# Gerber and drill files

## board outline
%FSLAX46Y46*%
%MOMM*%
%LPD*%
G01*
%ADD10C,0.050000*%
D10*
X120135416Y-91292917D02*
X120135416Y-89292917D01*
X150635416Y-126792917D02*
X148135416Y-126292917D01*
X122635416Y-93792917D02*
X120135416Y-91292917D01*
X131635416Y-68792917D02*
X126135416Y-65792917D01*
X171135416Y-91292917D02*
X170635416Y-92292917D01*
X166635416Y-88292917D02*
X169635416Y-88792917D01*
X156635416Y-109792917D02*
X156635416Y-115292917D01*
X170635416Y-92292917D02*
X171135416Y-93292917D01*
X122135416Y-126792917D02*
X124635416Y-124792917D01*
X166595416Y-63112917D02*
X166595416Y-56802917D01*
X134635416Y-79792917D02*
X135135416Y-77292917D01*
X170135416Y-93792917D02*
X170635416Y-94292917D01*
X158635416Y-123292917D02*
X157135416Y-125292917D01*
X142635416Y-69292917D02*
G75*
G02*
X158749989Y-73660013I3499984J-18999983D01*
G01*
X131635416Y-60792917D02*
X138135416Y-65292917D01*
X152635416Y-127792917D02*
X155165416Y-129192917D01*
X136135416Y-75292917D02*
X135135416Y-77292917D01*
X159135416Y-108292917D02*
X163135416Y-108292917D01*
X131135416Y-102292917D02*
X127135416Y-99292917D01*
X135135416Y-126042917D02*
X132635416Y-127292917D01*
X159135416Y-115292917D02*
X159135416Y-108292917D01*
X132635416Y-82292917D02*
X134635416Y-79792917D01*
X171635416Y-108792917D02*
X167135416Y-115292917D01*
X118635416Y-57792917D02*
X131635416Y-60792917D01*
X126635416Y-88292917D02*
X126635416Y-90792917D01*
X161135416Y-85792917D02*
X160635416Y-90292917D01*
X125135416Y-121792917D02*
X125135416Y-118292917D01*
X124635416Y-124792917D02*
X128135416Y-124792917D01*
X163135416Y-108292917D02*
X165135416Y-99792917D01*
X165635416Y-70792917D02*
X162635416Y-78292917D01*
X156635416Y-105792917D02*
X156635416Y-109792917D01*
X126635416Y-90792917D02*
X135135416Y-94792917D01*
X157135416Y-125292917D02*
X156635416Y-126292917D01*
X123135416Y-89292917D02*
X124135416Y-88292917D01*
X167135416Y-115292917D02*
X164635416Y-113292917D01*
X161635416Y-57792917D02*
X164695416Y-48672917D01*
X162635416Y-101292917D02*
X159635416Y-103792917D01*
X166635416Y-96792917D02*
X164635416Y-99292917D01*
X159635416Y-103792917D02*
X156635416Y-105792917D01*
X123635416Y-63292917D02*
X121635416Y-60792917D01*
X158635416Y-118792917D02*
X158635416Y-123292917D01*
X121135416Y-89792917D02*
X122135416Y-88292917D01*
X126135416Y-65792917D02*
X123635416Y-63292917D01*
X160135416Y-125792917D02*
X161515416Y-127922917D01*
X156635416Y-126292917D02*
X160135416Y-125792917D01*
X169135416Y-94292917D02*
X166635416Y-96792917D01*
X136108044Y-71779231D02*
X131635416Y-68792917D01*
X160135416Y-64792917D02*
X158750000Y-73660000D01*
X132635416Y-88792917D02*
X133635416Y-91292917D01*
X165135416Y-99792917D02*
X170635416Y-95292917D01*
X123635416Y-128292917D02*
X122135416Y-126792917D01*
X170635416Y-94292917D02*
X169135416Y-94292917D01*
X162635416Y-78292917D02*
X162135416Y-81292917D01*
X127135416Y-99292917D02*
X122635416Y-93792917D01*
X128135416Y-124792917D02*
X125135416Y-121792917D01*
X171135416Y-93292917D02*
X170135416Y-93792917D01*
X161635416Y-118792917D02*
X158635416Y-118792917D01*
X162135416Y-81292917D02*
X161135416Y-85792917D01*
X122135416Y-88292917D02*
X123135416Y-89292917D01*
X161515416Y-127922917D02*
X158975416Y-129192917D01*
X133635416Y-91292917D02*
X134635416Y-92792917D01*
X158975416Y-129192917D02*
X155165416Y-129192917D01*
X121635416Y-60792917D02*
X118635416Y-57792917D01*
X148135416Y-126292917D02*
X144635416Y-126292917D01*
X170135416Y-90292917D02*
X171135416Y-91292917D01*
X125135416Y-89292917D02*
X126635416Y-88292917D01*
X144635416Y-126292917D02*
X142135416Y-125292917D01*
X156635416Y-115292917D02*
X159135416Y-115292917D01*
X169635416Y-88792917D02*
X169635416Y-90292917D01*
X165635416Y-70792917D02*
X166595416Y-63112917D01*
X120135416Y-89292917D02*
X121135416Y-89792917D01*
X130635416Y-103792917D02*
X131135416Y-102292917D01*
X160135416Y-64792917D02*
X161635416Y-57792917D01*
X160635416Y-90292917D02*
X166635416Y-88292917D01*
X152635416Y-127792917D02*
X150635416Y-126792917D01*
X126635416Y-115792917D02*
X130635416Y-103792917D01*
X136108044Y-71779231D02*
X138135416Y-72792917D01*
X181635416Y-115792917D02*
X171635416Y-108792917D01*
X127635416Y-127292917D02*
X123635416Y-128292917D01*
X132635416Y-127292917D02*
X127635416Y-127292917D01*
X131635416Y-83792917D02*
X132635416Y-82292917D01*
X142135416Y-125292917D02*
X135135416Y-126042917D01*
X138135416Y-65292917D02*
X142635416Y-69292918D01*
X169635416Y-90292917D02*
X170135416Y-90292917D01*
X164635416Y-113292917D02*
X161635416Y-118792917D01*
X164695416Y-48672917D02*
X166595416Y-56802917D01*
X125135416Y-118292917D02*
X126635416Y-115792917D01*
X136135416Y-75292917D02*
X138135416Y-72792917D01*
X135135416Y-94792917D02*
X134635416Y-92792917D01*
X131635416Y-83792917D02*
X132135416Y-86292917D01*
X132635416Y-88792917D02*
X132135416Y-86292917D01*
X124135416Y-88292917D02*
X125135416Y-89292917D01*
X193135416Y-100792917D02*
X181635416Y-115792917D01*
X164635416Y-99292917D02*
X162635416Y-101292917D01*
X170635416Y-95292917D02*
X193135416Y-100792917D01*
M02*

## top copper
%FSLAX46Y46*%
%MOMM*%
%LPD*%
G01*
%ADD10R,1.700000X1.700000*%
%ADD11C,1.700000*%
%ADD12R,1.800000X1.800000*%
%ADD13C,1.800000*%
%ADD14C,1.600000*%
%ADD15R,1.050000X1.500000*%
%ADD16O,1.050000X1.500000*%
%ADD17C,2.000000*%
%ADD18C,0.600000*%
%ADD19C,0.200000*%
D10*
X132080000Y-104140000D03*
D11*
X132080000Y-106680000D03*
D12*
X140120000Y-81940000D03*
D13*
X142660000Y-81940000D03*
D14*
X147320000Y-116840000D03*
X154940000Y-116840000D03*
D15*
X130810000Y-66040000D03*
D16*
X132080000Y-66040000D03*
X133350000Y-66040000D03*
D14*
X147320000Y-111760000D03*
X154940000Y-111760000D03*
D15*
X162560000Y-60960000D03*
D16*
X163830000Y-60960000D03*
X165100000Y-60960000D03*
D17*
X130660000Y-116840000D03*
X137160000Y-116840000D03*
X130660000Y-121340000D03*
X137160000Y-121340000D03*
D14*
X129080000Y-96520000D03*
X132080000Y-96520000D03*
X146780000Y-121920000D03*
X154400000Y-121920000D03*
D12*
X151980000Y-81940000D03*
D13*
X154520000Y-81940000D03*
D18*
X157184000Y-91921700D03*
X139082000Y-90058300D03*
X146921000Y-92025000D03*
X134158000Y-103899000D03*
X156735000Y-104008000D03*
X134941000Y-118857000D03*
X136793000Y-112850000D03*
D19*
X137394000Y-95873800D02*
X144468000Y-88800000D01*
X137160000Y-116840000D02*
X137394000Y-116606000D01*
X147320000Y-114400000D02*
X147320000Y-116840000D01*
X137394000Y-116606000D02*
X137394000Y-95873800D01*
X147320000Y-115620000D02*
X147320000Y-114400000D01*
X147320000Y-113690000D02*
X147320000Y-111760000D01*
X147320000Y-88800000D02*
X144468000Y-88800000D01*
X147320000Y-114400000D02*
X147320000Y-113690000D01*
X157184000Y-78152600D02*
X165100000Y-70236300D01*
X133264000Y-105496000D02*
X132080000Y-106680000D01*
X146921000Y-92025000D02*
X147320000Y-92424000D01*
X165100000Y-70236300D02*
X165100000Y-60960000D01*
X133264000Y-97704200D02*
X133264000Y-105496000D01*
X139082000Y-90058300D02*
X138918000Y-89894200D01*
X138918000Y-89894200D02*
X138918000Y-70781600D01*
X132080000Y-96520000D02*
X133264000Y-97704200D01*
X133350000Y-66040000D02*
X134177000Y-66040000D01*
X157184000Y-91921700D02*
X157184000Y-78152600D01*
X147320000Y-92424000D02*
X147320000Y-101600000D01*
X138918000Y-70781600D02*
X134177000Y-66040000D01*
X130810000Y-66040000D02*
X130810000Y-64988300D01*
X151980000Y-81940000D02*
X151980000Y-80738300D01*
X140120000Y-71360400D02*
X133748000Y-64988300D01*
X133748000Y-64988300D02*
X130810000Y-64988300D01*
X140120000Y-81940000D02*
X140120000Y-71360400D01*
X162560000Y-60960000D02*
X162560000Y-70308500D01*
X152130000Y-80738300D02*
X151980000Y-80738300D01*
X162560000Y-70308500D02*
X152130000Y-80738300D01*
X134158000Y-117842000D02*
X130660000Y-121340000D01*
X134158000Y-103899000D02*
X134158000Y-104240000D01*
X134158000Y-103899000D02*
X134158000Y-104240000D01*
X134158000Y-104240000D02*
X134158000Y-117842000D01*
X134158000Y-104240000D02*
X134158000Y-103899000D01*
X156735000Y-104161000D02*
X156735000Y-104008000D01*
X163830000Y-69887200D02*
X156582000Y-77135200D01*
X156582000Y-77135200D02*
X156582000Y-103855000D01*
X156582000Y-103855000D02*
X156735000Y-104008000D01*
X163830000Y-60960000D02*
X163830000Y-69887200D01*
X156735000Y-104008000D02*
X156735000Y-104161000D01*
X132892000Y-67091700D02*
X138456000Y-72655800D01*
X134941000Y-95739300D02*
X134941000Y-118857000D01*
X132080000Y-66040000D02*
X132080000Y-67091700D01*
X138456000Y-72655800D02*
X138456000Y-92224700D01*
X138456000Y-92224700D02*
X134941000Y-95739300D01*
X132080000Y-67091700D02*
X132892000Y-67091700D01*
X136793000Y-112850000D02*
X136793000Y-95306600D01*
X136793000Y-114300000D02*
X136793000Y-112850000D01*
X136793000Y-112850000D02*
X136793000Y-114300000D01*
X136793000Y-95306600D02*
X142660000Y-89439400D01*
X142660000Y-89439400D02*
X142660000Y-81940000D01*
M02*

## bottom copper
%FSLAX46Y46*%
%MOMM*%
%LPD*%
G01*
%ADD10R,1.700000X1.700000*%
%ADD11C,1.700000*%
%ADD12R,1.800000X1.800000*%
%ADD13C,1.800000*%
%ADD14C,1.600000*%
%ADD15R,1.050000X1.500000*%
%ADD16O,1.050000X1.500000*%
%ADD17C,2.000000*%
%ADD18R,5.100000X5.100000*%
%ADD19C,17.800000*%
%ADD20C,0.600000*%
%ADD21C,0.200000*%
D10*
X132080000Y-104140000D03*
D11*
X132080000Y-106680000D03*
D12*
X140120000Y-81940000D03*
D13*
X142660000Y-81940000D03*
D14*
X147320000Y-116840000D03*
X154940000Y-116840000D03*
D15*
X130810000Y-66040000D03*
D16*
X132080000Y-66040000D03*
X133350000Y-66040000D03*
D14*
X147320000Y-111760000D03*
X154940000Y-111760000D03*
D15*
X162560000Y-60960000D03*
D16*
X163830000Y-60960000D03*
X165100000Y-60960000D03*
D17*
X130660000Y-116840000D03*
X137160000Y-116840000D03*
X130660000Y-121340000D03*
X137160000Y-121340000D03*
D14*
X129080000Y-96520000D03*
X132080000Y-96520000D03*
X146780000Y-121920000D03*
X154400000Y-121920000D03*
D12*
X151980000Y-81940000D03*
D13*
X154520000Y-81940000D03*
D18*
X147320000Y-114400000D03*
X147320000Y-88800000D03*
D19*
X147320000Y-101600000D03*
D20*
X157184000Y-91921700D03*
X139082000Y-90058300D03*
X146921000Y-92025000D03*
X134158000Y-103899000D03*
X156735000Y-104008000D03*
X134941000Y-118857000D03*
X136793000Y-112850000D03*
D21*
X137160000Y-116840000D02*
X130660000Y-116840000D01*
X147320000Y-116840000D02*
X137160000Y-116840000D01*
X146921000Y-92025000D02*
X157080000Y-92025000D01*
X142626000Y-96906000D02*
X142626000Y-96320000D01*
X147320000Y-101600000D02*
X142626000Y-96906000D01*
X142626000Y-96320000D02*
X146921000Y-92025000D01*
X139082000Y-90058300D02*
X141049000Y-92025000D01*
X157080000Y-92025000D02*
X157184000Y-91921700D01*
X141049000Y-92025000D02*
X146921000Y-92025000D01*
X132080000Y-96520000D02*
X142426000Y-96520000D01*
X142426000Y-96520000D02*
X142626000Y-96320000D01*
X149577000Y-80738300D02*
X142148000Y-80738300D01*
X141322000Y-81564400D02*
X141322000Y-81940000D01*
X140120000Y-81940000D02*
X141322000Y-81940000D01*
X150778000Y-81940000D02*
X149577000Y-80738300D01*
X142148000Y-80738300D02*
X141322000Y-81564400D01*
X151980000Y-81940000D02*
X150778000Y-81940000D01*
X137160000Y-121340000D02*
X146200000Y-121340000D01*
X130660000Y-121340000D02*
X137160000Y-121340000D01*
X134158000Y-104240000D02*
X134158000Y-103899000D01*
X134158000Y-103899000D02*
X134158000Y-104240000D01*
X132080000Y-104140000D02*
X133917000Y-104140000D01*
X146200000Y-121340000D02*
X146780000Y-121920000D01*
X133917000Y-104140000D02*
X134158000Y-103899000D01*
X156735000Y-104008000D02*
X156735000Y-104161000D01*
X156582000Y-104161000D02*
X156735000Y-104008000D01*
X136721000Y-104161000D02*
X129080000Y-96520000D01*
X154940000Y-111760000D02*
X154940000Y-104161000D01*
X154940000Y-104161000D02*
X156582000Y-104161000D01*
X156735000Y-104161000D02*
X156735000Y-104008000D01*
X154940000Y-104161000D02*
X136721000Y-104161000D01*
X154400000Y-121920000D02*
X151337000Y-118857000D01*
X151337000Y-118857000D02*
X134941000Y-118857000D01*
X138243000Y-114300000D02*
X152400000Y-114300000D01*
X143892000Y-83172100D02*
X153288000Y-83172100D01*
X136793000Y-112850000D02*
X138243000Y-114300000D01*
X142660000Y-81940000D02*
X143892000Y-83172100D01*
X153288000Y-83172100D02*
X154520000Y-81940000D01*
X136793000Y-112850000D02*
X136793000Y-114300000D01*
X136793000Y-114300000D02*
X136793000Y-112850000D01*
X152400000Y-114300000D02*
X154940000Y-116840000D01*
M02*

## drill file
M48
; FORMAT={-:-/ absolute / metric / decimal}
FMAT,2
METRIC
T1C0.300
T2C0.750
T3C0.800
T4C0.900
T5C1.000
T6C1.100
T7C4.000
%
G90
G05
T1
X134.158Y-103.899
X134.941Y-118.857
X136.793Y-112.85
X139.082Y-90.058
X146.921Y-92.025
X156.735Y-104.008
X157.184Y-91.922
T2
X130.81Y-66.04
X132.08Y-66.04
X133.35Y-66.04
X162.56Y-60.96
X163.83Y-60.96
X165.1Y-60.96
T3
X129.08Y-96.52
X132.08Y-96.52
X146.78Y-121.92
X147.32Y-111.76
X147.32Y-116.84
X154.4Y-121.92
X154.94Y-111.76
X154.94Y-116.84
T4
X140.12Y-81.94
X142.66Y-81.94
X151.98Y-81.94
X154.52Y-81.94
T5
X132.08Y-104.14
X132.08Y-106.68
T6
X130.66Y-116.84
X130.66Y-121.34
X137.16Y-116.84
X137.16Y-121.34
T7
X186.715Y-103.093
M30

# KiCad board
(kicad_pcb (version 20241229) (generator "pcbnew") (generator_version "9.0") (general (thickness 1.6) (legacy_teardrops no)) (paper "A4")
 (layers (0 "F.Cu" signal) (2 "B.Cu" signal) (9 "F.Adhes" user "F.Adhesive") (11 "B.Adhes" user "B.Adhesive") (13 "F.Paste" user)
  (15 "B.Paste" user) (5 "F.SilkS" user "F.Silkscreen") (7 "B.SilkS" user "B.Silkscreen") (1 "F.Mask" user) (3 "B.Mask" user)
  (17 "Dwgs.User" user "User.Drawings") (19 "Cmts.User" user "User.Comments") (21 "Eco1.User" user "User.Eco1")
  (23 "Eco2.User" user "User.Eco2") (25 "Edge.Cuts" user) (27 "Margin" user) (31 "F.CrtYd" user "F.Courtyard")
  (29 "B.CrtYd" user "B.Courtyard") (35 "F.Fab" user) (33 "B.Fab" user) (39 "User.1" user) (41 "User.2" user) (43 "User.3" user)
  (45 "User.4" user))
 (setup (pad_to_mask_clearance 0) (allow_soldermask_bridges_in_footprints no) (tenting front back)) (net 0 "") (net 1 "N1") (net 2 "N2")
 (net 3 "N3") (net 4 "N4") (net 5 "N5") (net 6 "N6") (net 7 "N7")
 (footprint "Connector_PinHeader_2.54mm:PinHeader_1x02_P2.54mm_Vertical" (layer "F.Cu") (at 132.08 104.14)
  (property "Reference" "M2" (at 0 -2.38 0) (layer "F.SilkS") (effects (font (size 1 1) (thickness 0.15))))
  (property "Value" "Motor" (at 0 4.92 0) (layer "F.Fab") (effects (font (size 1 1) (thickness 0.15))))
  (pad "1" thru_hole rect (at 0 0) (size 1.7 1.7) (drill 1) (layers "*.Cu" "*.Mask") (remove_unused_layers no) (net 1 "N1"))
  (pad "2" thru_hole circle (at 0 2.54) (size 1.7 1.7) (drill 1) (layers "*.Cu" "*.Mask") (remove_unused_layers no) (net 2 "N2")))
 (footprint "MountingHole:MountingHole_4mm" (layer "F.Cu") (at 186.7154 103.0929)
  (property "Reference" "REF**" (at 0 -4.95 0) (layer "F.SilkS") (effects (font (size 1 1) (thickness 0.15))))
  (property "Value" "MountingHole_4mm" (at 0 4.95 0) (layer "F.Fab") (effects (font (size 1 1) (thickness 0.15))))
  (pad "" np_thru_hole circle (at 0 0) (size 4 4) (drill 4) (layers "*.Cu" "*.Mask")))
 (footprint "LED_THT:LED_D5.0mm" (layer "F.Cu") (at 140.12 81.94)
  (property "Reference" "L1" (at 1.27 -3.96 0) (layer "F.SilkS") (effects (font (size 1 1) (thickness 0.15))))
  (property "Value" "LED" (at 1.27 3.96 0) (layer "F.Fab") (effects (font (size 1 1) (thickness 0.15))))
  (pad "1" thru_hole rect (at 0 0) (size 1.8 1.8) (drill 0.9) (layers "*.Cu" "*.Mask") (remove_unused_layers no) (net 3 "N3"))
  (pad "2" thru_hole circle (at 2.54 0) (size 1.8 1.8) (drill 0.9) (layers "*.Cu" "*.Mask") (remove_unused_layers no) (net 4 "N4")))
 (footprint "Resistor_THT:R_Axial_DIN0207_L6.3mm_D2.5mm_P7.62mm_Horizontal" (layer "F.Cu") (at 147.32 116.84)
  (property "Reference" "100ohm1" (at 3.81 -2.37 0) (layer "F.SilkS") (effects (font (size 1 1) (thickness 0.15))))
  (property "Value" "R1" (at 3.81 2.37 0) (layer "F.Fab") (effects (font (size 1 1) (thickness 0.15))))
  (pad "1" thru_hole circle (at 0 0) (size 1.6 1.6) (drill 0.8) (layers "*.Cu" "*.Mask") (remove_unused_layers no) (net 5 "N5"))
  (pad "2" thru_hole circle (at 7.62 0) (size 1.6 1.6) (drill 0.8) (layers "*.Cu" "*.Mask") (remove_unused_layers no) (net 4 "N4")))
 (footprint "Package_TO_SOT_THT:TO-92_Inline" (layer "F.Cu") (at 130.81 66.04)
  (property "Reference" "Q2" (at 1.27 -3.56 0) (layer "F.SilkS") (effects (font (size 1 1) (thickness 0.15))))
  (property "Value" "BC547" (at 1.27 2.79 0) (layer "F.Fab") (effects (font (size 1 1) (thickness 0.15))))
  (pad "1" thru_hole rect (at 0 0) (size 1.05 1.5) (drill 0.75) (layers "*.Cu" "*.Mask") (remove_unused_layers no) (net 3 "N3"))
  (pad "2" thru_hole oval (at 1.27 0) (size 1.05 1.5) (drill 0.75) (layers "*.Cu" "*.Mask") (remove_unused_layers no) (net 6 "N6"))
  (pad "3" thru_hole oval (at 2.54 0) (size 1.05 1.5) (drill 0.75) (layers "*.Cu" "*.Mask") (remove_unused_layers no) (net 2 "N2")))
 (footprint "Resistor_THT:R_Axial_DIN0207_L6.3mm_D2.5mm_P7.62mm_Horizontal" (layer "F.Cu") (at 147.32 111.76)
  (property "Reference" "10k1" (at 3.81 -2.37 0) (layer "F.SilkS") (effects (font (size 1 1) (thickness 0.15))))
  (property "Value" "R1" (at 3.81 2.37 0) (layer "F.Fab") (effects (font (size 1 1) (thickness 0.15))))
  (pad "1" thru_hole circle (at 0 0) (size 1.6 1.6) (drill 0.8) (layers "*.Cu" "*.Mask") (remove_unused_layers no) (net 5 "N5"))
  (pad "2" thru_hole circle (at 7.62 0) (size 1.6 1.6) (drill 0.8) (layers "*.Cu" "*.Mask") (remove_unused_layers no) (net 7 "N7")))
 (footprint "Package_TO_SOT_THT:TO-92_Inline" (layer "F.Cu") (at 162.56 60.96)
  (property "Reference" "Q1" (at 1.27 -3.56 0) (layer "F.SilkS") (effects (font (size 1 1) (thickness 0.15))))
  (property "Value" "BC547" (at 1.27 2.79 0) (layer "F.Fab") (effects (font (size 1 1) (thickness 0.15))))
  (pad "1" thru_hole rect (at 0 0) (size 1.05 1.5) (drill 0.75) (layers "*.Cu" "*.Mask") (remove_unused_layers no) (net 3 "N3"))
  (pad "2" thru_hole oval (at 1.27 0) (size 1.05 1.5) (drill 0.75) (layers "*.Cu" "*.Mask") (remove_unused_layers no) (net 7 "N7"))
  (pad "3" thru_hole oval (at 2.54 0) (size 1.05 1.5) (drill 0.75) (layers "*.Cu" "*.Mask") (remove_unused_layers no) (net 2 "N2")))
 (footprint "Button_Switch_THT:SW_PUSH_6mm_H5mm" (layer "F.Cu") (at 130.66 116.84)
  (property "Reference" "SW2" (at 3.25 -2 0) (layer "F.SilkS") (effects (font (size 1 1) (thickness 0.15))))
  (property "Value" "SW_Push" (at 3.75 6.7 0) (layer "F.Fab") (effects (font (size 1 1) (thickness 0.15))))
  (pad "1" thru_hole circle (at 0 0 90) (size 2 2) (drill 1.1) (layers "*.Cu" "*.Mask") (remove_unused_layers no) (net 5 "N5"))
  (pad "1" thru_hole circle (at 6.5 0 90) (size 2 2) (drill 1.1) (layers "*.Cu" "*.Mask") (remove_unused_layers no) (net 5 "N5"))
  (pad "2" thru_hole circle (at 0 4.5 90) (size 2 2) (drill 1.1) (layers "*.Cu" "*.Mask") (remove_unused_layers no) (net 1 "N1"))
  (pad "2" thru_hole circle (at 6.5 4.5 90) (size 2 2) (drill 1.1) (layers "*.Cu" "*.Mask") (remove_unused_layers no) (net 1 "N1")))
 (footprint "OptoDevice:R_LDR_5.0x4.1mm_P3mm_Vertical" (layer "F.Cu") (at 129.08 96.52)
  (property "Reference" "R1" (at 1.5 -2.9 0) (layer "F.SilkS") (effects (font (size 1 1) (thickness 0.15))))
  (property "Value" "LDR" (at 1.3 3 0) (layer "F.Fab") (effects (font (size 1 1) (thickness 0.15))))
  (pad "1" thru_hole circle (at 0 0) (size 1.6 1.6) (drill 0.8) (layers "*.Cu" "*.Mask") (remove_unused_layers no) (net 7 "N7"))
  (pad "2" thru_hole circle (at 3 0) (size 1.6 1.6) (drill 0.8) (layers "*.Cu" "*.Mask") (remove_unused_layers no) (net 2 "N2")))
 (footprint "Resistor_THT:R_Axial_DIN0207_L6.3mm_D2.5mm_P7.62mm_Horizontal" (layer "F.Cu") (at 146.78 121.92)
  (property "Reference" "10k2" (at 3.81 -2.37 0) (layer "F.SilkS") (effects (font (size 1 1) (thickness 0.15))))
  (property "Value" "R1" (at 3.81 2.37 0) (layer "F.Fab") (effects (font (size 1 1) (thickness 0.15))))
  (pad "1" thru_hole circle (at 0 0) (size 1.6 1.6) (drill 0.8) (layers "*.Cu" "*.Mask") (remove_unused_layers no) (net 1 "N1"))
  (pad "2" thru_hole circle (at 7.62 0) (size 1.6 1.6) (drill 0.8) (layers "*.Cu" "*.Mask") (remove_unused_layers no) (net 6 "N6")))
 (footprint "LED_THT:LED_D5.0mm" (layer "F.Cu") (at 151.98 81.94)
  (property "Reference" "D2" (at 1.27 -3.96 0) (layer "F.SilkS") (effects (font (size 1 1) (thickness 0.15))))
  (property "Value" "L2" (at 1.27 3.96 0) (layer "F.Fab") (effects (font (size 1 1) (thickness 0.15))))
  (pad "1" thru_hole rect (at 0 0) (size 1.8 1.8) (drill 0.9) (layers "*.Cu" "*.Mask") (remove_unused_layers no) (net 3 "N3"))
  (pad "2" thru_hole circle (at 2.54 0) (size 1.8 1.8) (drill 0.9) (layers "*.Cu" "*.Mask") (remove_unused_layers no) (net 4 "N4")))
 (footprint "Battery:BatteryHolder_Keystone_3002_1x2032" (layer "B.Cu") (at 147.32 101.6 90)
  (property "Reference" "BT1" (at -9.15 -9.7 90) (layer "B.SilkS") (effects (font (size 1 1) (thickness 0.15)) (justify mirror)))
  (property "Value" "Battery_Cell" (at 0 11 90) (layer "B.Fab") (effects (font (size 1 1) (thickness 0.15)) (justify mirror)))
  (pad "1" smd rect (at -12.8 0 90) (size 5.1 5.1) (layers "B.Cu" "B.Mask" "B.Paste") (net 5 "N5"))
  (pad "1" smd rect (at 12.8 0 90) (size 5.1 5.1) (layers "B.Cu" "B.Mask" "B.Paste") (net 5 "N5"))
  (pad "2" smd circle (at 0 0 90) (size 17.8 17.8) (layers "B.Cu" "B.Mask") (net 2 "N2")))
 (gr_line (start 120.135416 91.292917) (end 120.135416 89.292917) (stroke (width 0.05) (type default)) (layer "Edge.Cuts"))
 (gr_line (start 150.635416 126.792917) (end 148.135416 126.292917) (stroke (width 0.05) (type default)) (layer "Edge.Cuts"))
 (gr_line (start 122.635416 93.792917) (end 120.135416 91.292917) (stroke (width 0.05) (type default)) (layer "Edge.Cuts"))
 (gr_line (start 131.635416 68.792917) (end 126.135416 65.792917) (stroke (width 0.05) (type default)) (layer "Edge.Cuts"))
 (gr_line (start 171.135416 91.292917) (end 170.635416 92.292917) (stroke (width 0.05) (type default)) (layer "Edge.Cuts"))
 (gr_line (start 166.635416 88.292917) (end 169.635416 88.792917) (stroke (width 0.05) (type default)) (layer "Edge.Cuts"))
 (gr_line (start 156.635416 109.792917) (end 156.635416 115.292917) (stroke (width 0.05) (type default)) (layer "Edge.Cuts"))
 (gr_line (start 170.635416 92.292917) (end 171.135416 93.292917) (stroke (width 0.05) (type default)) (layer "Edge.Cuts"))
 (gr_line (start 122.135416 126.792917) (end 124.635416 124.792917) (stroke (width 0.05) (type default)) (layer "Edge.Cuts"))
 (gr_line (start 166.595416 63.112917) (end 166.595416 56.802917) (stroke (width 0.05) (type default)) (layer "Edge.Cuts"))
 (gr_line (start 134.635416 79.792917) (end 135.135416 77.292917) (stroke (width 0.05) (type default)) (layer "Edge.Cuts"))
 (gr_line (start 170.135416 93.792917) (end 170.635416 94.292917) (stroke (width 0.05) (type default)) (layer "Edge.Cuts"))
 (gr_line (start 158.635416 123.292917) (end 157.135416 125.292917) (stroke (width 0.05) (type default)) (layer "Edge.Cuts"))
 (gr_arc (start 142.635416 69.292917) (mid 151.188807 69.645847) (end 158.75 73.66) (stroke (width 0.05) (type default)) (layer "Edge.Cuts"))
 (gr_line (start 131.635416 60.792917) (end 138.135416 65.292917) (stroke (width 0.05) (type default)) (layer "Edge.Cuts"))
 (gr_line (start 152.635416 127.792917) (end 155.165416 129.192917) (stroke (width 0.05) (type default)) (layer "Edge.Cuts"))
 (gr_line (start 136.135416 75.292917) (end 135.135416 77.292917) (stroke (width 0.05) (type default)) (layer "Edge.Cuts"))
 (gr_line (start 159.135416 108.292917) (end 163.135416 108.292917) (stroke (width 0.05) (type default)) (layer "Edge.Cuts"))
 (gr_line (start 131.135416 102.292917) (end 127.135416 99.292917) (stroke (width 0.05) (type default)) (layer "Edge.Cuts"))
 (gr_line (start 135.135416 126.042917) (end 132.635416 127.292917) (stroke (width 0.05) (type default)) (layer "Edge.Cuts"))
 (gr_line (start 159.135416 115.292917) (end 159.135416 108.292917) (stroke (width 0.05) (type default)) (layer "Edge.Cuts"))
 (gr_line (start 132.635416 82.292917) (end 134.635416 79.792917) (stroke (width 0.05) (type default)) (layer "Edge.Cuts"))
 (gr_line (start 171.635416 108.792917) (end 167.135416 115.292917) (stroke (width 0.05) (type default)) (layer "Edge.Cuts"))
 (gr_line (start 118.635416 57.792917) (end 131.635416 60.792917) (stroke (width 0.05) (type default)) (layer "Edge.Cuts"))
 (gr_line (start 126.635416 88.292917) (end 126.635416 90.792917) (stroke (width 0.05) (type default)) (layer "Edge.Cuts"))
 (gr_line (start 161.135416 85.792917) (end 160.635416 90.292917) (stroke (width 0.05) (type default)) (layer "Edge.Cuts"))
 (gr_line (start 125.135416 121.792917) (end 125.135416 118.292917) (stroke (width 0.05) (type default)) (layer "Edge.Cuts"))
 (gr_line (start 124.635416 124.792917) (end 128.135416 124.792917) (stroke (width 0.05) (type default)) (layer "Edge.Cuts"))
 (gr_line (start 163.135416 108.292917) (end 165.135416 99.792917) (stroke (width 0.05) (type default)) (layer "Edge.Cuts"))
 (gr_line (start 165.635416 70.792917) (end 162.635416 78.292917) (stroke (width 0.05) (type default)) (layer "Edge.Cuts"))
 (gr_line (start 156.635416 105.792917) (end 156.635416 109.792917) (stroke (width 0.05) (type default)) (layer "Edge.Cuts"))
 (gr_line (start 126.635416 90.792917) (end 135.135416 94.792917) (stroke (width 0.05) (type default)) (layer "Edge.Cuts"))
 (gr_line (start 157.135416 125.292917) (end 156.635416 126.292917) (stroke (width 0.05) (type default)) (layer "Edge.Cuts"))
 (gr_line (start 123.135416 89.292917) (end 124.135416 88.292917) (stroke (width 0.05) (type default)) (layer "Edge.Cuts"))
 (gr_line (start 167.135416 115.292917) (end 164.635416 113.292917) (stroke (width 0.05) (type default)) (layer "Edge.Cuts"))
 (gr_line (start 161.635416 57.792917) (end 164.695416 48.672917) (stroke (width 0.05) (type default)) (layer "Edge.Cuts"))
 (gr_line (start 162.635416 101.292917) (end 159.635416 103.792917) (stroke (width 0.05) (type default)) (layer "Edge.Cuts"))
 (gr_line (start 166.635416 96.792917) (end 164.635416 99.292917) (stroke (width 0.05) (type default)) (layer "Edge.Cuts"))
 (gr_line (start 159.635416 103.792917) (end 156.635416 105.792917) (stroke (width 0.05) (type default)) (layer "Edge.Cuts"))
 (gr_line (start 123.635416 63.292917) (end 121.635416 60.792917) (stroke (width 0.05) (type default)) (layer "Edge.Cuts"))
 (gr_line (start 158.635416 118.792917) (end 158.635416 123.292917) (stroke (width 0.05) (type default)) (layer "Edge.Cuts"))
 (gr_line (start 121.135416 89.792917) (end 122.135416 88.292917) (stroke (width 0.05) (type default)) (layer "Edge.Cuts"))
 (gr_line (start 126.135416 65.792917) (end 123.635416 63.292917) (stroke (width 0.05) (type default)) (layer "Edge.Cuts"))
 (gr_line (start 160.135416 125.792917) (end 161.515416 127.922917) (stroke (width 0.05) (type default)) (layer "Edge.Cuts"))
 (gr_line (start 156.635416 126.292917) (end 160.135416 125.792917) (stroke (width 0.05) (type default)) (layer "Edge.Cuts"))
 (gr_line (start 169.135416 94.292917) (end 166.635416 96.792917) (stroke (width 0.05) (type default)) (layer "Edge.Cuts"))
 (gr_line (start 136.108044 71.779231) (end 131.635416 68.792917) (stroke (width 0.05) (type default)) (layer "Edge.Cuts"))
 (gr_line (start 160.135416 64.792917) (end 158.75 73.66) (stroke (width 0.05) (type default)) (layer "Edge.Cuts"))
 (gr_line (start 132.635416 88.792917) (end 133.635416 91.292917) (stroke (width 0.05) (type default)) (layer "Edge.Cuts"))
 (gr_line (start 165.135416 99.792917) (end 170.635416 95.292917) (stroke (width 0.05) (type default)) (layer "Edge.Cuts"))
 (gr_line (start 123.635416 128.292917) (end 122.135416 126.792917) (stroke (width 0.05) (type default)) (layer "Edge.Cuts"))
 (gr_line (start 170.635416 94.292917) (end 169.135416 94.292917) (stroke (width 0.05) (type default)) (layer "Edge.Cuts"))
 (gr_line (start 162.635416 78.292917) (end 162.135416 81.292917) (stroke (width 0.05) (type default)) (layer "Edge.Cuts"))
 (gr_line (start 127.135416 99.292917) (end 122.635416 93.792917) (stroke (width 0.05) (type default)) (layer "Edge.Cuts"))
 (gr_line (start 128.135416 124.792917) (end 125.135416 121.792917) (stroke (width 0.05) (type default)) (layer "Edge.Cuts"))
 (gr_line (start 171.135416 93.292917) (end 170.135416 93.792917) (stroke (width 0.05) (type default)) (layer "Edge.Cuts"))
 (gr_line (start 161.635416 118.792917) (end 158.635416 118.792917) (stroke (width 0.05) (type default)) (layer "Edge.Cuts"))
 (gr_line (start 162.135416 81.292917) (end 161.135416 85.792917) (stroke (width 0.05) (type default)) (layer "Edge.Cuts"))
 (gr_line (start 122.135416 88.292917) (end 123.135416 89.292917) (stroke (width 0.05) (type default)) (layer "Edge.Cuts"))
 (gr_line (start 161.515416 127.922917) (end 158.975416 129.192917) (stroke (width 0.05) (type default)) (layer "Edge.Cuts"))
 (gr_line (start 133.635416 91.292917) (end 134.635416 92.792917) (stroke (width 0.05) (type default)) (layer "Edge.Cuts"))
 (gr_line (start 158.975416 129.192917) (end 155.165416 129.192917) (stroke (width 0.05) (type default)) (layer "Edge.Cuts"))
 (gr_line (start 121.635416 60.792917) (end 118.635416 57.792917) (stroke (width 0.05) (type default)) (layer "Edge.Cuts"))
 (gr_line (start 148.135416 126.292917) (end 144.635416 126.292917) (stroke (width 0.05) (type default)) (layer "Edge.Cuts"))
 (gr_line (start 170.135416 90.292917) (end 171.135416 91.292917) (stroke (width 0.05) (type default)) (layer "Edge.Cuts"))
 (gr_line (start 125.135416 89.292917) (end 126.635416 88.292917) (stroke (width 0.05) (type default)) (layer "Edge.Cuts"))
 (gr_line (start 144.635416 126.292917) (end 142.135416 125.292917) (stroke (width 0.05) (type default)) (layer "Edge.Cuts"))
 (gr_line (start 156.635416 115.292917) (end 159.135416 115.292917) (stroke (width 0.05) (type default)) (layer "Edge.Cuts"))
 (gr_line (start 169.635416 88.792917) (end 169.635416 90.292917) (stroke (width 0.05) (type default)) (layer "Edge.Cuts"))
 (gr_line (start 165.635416 70.792917) (end 166.595416 63.112917) (stroke (width 0.05) (type default)) (layer "Edge.Cuts"))
 (gr_line (start 120.135416 89.292917) (end 121.135416 89.792917) (stroke (width 0.05) (type default)) (layer "Edge.Cuts"))
 (gr_line (start 130.635416 103.792917) (end 131.135416 102.292917) (stroke (width 0.05) (type default)) (layer "Edge.Cuts"))
 (gr_line (start 160.135416 64.792917) (end 161.635416 57.792917) (stroke (width 0.05) (type default)) (layer "Edge.Cuts"))
 (gr_line (start 160.635416 90.292917) (end 166.635416 88.292917) (stroke (width 0.05) (type default)) (layer "Edge.Cuts"))
 (gr_line (start 152.635416 127.792917) (end 150.635416 126.792917) (stroke (width 0.05) (type default)) (layer "Edge.Cuts"))
 (gr_line (start 126.635416 115.792917) (end 130.635416 103.792917) (stroke (width 0.05) (type default)) (layer "Edge.Cuts"))
 (gr_line (start 136.108044 71.779231) (end 138.135416 72.792917) (stroke (width 0.05) (type default)) (layer "Edge.Cuts"))
 (gr_line (start 181.635416 115.792917) (end 171.635416 108.792917) (stroke (width 0.05) (type default)) (layer "Edge.Cuts"))
 (gr_line (start 127.635416 127.292917) (end 123.635416 128.292917) (stroke (width 0.05) (type default)) (layer "Edge.Cuts"))
 (gr_line (start 132.635416 127.292917) (end 127.635416 127.292917) (stroke (width 0.05) (type default)) (layer "Edge.Cuts"))
 (gr_line (start 131.635416 83.792917) (end 132.635416 82.292917) (stroke (width 0.05) (type default)) (layer "Edge.Cuts"))
 (gr_line (start 142.135416 125.292917) (end 135.135416 126.042917) (stroke (width 0.05) (type default)) (layer "Edge.Cuts"))
 (gr_line (start 138.135416 65.292917) (end 142.635416 69.292918) (stroke (width 0.05) (type default)) (layer "Edge.Cuts"))
 (gr_line (start 169.635416 90.292917) (end 170.135416 90.292917) (stroke (width 0.05) (type default)) (layer "Edge.Cuts"))
 (gr_line (start 164.635416 113.292917) (end 161.635416 118.792917) (stroke (width 0.05) (type default)) (layer "Edge.Cuts"))
 (gr_line (start 164.695416 48.672917) (end 166.595416 56.802917) (stroke (width 0.05) (type default)) (layer "Edge.Cuts"))
 (gr_line (start 125.135416 118.292917) (end 126.635416 115.792917) (stroke (width 0.05) (type default)) (layer "Edge.Cuts"))
 (gr_line (start 136.135416 75.292917) (end 138.135416 72.792917) (stroke (width 0.05) (type default)) (layer "Edge.Cuts"))
 (gr_line (start 135.135416 94.792917) (end 134.635416 92.792917) (stroke (width 0.05) (type default)) (layer "Edge.Cuts"))
 (gr_line (start 131.635416 83.792917) (end 132.135416 86.292917) (stroke (width 0.05) (type default)) (layer "Edge.Cuts"))
 (gr_line (start 132.635416 88.792917) (end 132.135416 86.292917) (stroke (width 0.05) (type default)) (layer "Edge.Cuts"))
 (gr_line (start 124.135416 88.292917) (end 125.135416 89.292917) (stroke (width 0.05) (type default)) (layer "Edge.Cuts"))
 (gr_line (start 193.135416 100.792917) (end 181.635416 115.792917) (stroke (width 0.05) (type default)) (layer "Edge.Cuts"))
 (gr_line (start 164.635416 99.292917) (end 162.635416 101.292917) (stroke (width 0.05) (type default)) (layer "Edge.Cuts"))
 (gr_line (start 170.635416 95.292917) (end 193.135416 100.792917) (stroke (width 0.05) (type default)) (layer "Edge.Cuts"))
 (segment (start 137.394 95.8738) (end 144.468 88.8) (width 0.2) (layer "F.Cu") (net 5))
 (segment (start 137.16 116.84) (end 137.394 116.606) (width 0.2) (layer "F.Cu") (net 5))
 (segment (start 147.32 114.4) (end 147.32 116.84) (width 0.2) (layer "F.Cu") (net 5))
 (segment (start 137.394 116.606) (end 137.394 95.8738) (width 0.2) (layer "F.Cu") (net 5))
 (segment (start 147.32 115.62) (end 147.32 114.4) (width 0.2) (layer "F.Cu") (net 5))
 (segment (start 147.32 113.69) (end 147.32 111.76) (width 0.2) (layer "F.Cu") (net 5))
 (segment (start 147.32 88.8) (end 144.468 88.8) (width 0.2) (layer "F.Cu") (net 5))
 (segment (start 147.32 114.4) (end 147.32 113.69) (width 0.2) (layer "F.Cu") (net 5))
 (segment (start 137.16 116.84) (end 130.66 116.84) (width 0.2) (layer "B.Cu") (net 5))
 (segment (start 147.32 116.84) (end 137.16 116.84) (width 0.2) (layer "B.Cu") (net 5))
 (segment (start 157.184 78.1526) (end 165.1 70.2363) (width 0.2) (layer "F.Cu") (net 2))
 (segment (start 133.264 105.496) (end 132.08 106.68) (width 0.2) (layer "F.Cu") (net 2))
 (segment (start 146.921 92.025) (end 147.32 92.424) (width 0.2) (layer "F.Cu") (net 2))
 (segment (start 165.1 70.2363) (end 165.1 60.96) (width 0.2) (layer "F.Cu") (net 2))
 (segment (start 133.264 97.7042) (end 133.264 105.496) (width 0.2) (layer "F.Cu") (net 2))
 (segment (start 139.082 90.0583) (end 138.918 89.8942) (width 0.2) (layer "F.Cu") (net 2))
 (segment (start 138.918 89.8942) (end 138.918 70.7816) (width 0.2) (layer "F.Cu") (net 2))
 (segment (start 132.08 96.52) (end 133.264 97.7042) (width 0.2) (layer "F.Cu") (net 2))
 (segment (start 133.35 66.04) (end 134.177 66.04) (width 0.2) (layer "F.Cu") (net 2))
 (segment (start 157.184 91.9217) (end 157.184 78.1526) (width 0.2) (layer "F.Cu") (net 2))
 (segment (start 147.32 92.424) (end 147.32 101.6) (width 0.2) (layer "F.Cu") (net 2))
 (segment (start 138.918 70.7816) (end 134.177 66.04) (width 0.2) (layer "F.Cu") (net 2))
 (via (at 157.184 91.9217) (size 0.6) (drill 0.3) (layers "F.Cu" "B.Cu") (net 2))
 (via (at 139.082 90.0583) (size 0.6) (drill 0.3) (layers "F.Cu" "B.Cu") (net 2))
 (via (at 146.921 92.025) (size 0.6) (drill 0.3) (layers "F.Cu" "B.Cu") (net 2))
 (segment (start 146.921 92.025) (end 157.08 92.025) (width 0.2) (layer "B.Cu") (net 2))
 (segment (start 142.626 96.906) (end 142.626 96.32) (width 0.2) (layer "B.Cu") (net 2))
 (segment (start 147.32 101.6) (end 142.626 96.906) (width 0.2) (layer "B.Cu") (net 2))
 (segment (start 142.626 96.32) (end 146.921 92.025) (width 0.2) (layer "B.Cu") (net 2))
 (segment (start 139.082 90.0583) (end 141.049 92.025) (width 0.2) (layer "B.Cu") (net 2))
 (segment (start 157.08 92.025) (end 157.184 91.9217) (width 0.2) (layer "B.Cu") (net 2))
 (segment (start 141.049 92.025) (end 146.921 92.025) (width 0.2) (layer "B.Cu") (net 2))
 (segment (start 132.08 96.52) (end 142.426 96.52) (width 0.2) (layer "B.Cu") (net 2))
 (segment (start 142.426 96.52) (end 142.626 96.32) (width 0.2) (layer "B.Cu") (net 2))
 (segment (start 130.81 66.04) (end 130.81 64.9883) (width 0.2) (layer "F.Cu") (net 3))
 (segment (start 151.98 81.94) (end 151.98 80.7383) (width 0.2) (layer "F.Cu") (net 3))
 (segment (start 140.12 71.3604) (end 133.748 64.9883) (width 0.2) (layer "F.Cu") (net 3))
 (segment (start 133.748 64.9883) (end 130.81 64.9883) (width 0.2) (layer "F.Cu") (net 3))
 (segment (start 140.12 81.94) (end 140.12 71.3604) (width 0.2) (layer "F.Cu") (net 3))
 (segment (start 162.56 60.96) (end 162.56 70.3085) (width 0.2) (layer "F.Cu") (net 3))
 (segment (start 152.13 80.7383) (end 151.98 80.7383) (width 0.2) (layer "F.Cu") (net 3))
 (segment (start 162.56 70.3085) (end 152.13 80.7383) (width 0.2) (layer "F.Cu") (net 3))
 (segment (start 149.577 80.7383) (end 142.148 80.7383) (width 0.2) (layer "B.Cu") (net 3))
 (segment (start 141.322 81.5644) (end 141.322 81.94) (width 0.2) (layer "B.Cu") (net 3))
 (segment (start 140.12 81.94) (end 141.322 81.94) (width 0.2) (layer "B.Cu") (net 3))
 (segment (start 150.778 81.94) (end 149.577 80.7383) (width 0.2) (layer "B.Cu") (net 3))
 (segment (start 142.148 80.7383) (end 141.322 81.5644) (width 0.2) (layer "B.Cu") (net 3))
 (segment (start 151.98 81.94) (end 150.778 81.94) (width 0.2) (layer "B.Cu") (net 3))
 (segment (start 134.158 117.842) (end 130.66 121.34) (width 0.2) (layer "F.Cu") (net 1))
 (segment (start 134.158 103.899) (end 134.158 104.24) (width 0.2) (layer "F.Cu") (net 1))
 (segment (start 134.158 103.899) (end 134.158 104.24) (width 0.2) (layer "F.Cu") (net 1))
 (segment (start 134.158 104.24) (end 134.158 117.842) (width 0.2) (layer "F.Cu") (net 1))
 (segment (start 134.158 104.24) (end 134.158 103.899) (width 0.2) (layer "F.Cu") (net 1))
 (via (at 134.158 103.899) (size 0.6) (drill 0.3) (layers "F.Cu" "B.Cu") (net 1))
 (segment (start 137.16 121.34) (end 146.2 121.34) (width 0.2) (layer "B.Cu") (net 1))
 (segment (start 130.66 121.34) (end 137.16 121.34) (width 0.2) (layer "B.Cu") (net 1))
 (segment (start 134.158 104.24) (end 134.158 103.899) (width 0.2) (layer "B.Cu") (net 1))
 (segment (start 134.158 103.899) (end 134.158 104.24) (width 0.2) (layer "B.Cu") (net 1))
 (segment (start 132.08 104.14) (end 133.917 104.14) (width 0.2) (layer "B.Cu") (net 1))
 (segment (start 146.2 121.34) (end 146.78 121.92) (width 0.2) (layer "B.Cu") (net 1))
 (segment (start 133.917 104.14) (end 134.158 103.899) (width 0.2) (layer "B.Cu") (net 1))
 (segment (start 156.735 104.161) (end 156.735 104.008) (width 0.2) (layer "F.Cu") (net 7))
 (segment (start 163.83 69.8872) (end 156.582 77.1352) (width 0.2) (layer "F.Cu") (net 7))
 (segment (start 156.582 77.1352) (end 156.582 103.855) (width 0.2) (layer "F.Cu") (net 7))
 (segment (start 156.582 103.855) (end 156.735 104.008) (width 0.2) (layer "F.Cu") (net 7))
 (segment (start 163.83 60.96) (end 163.83 69.8872) (width 0.2) (layer "F.Cu") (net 7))
 (segment (start 156.735 104.008) (end 156.735 104.161) (width 0.2) (layer "F.Cu") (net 7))
 (via (at 156.735 104.008) (size 0.6) (drill 0.3) (layers "F.Cu" "B.Cu") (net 7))
 (segment (start 156.735 104.008) (end 156.735 104.161) (width 0.2) (layer "B.Cu") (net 7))
 (segment (start 156.582 104.161) (end 156.735 104.008) (width 0.2) (layer "B.Cu") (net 7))
 (segment (start 136.721 104.161) (end 129.08 96.52) (width 0.2) (layer "B.Cu") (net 7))
 (segment (start 154.94 111.76) (end 154.94 104.161) (width 0.2) (layer "B.Cu") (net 7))
 (segment (start 154.94 104.161) (end 156.582 104.161) (width 0.2) (layer "B.Cu") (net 7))
 (segment (start 156.735 104.161) (end 156.735 104.008) (width 0.2) (layer "B.Cu") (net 7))
 (segment (start 154.94 104.161) (end 136.721 104.161) (width 0.2) (layer "B.Cu") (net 7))
 (segment (start 132.892 67.0917) (end 138.456 72.6558) (width 0.2) (layer "F.Cu") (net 6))
 (segment (start 134.941 95.7393) (end 134.941 118.857) (width 0.2) (layer "F.Cu") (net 6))
 (segment (start 132.08 66.04) (end 132.08 67.0917) (width 0.2) (layer "F.Cu") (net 6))
 (segment (start 138.456 72.6558) (end 138.456 92.2247) (width 0.2) (layer "F.Cu") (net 6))
 (segment (start 138.456 92.2247) (end 134.941 95.7393) (width 0.2) (layer "F.Cu") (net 6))
 (segment (start 132.08 67.0917) (end 132.892 67.0917) (width 0.2) (layer "F.Cu") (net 6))
 (via (at 134.941 118.857) (size 0.6) (drill 0.3) (layers "F.Cu" "B.Cu") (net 6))
 (segment (start 154.4 121.92) (end 151.337 118.857) (width 0.2) (layer "B.Cu") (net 6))
 (segment (start 151.337 118.857) (end 134.941 118.857) (width 0.2) (layer "B.Cu") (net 6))
 (segment (start 136.793 112.85) (end 136.793 95.3066) (width 0.2) (layer "F.Cu") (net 4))
 (segment (start 136.793 114.3) (end 136.793 112.85) (width 0.2) (layer "F.Cu") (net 4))
 (segment (start 136.793 112.85) (end 136.793 114.3) (width 0.2) (layer "F.Cu") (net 4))
 (segment (start 136.793 95.3066) (end 142.66 89.4394) (width 0.2) (layer "F.Cu") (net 4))
 (segment (start 142.66 89.4394) (end 142.66 81.94) (width 0.2) (layer "F.Cu") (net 4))
 (via (at 136.793 112.85) (size 0.6) (drill 0.3) (layers "F.Cu" "B.Cu") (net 4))
 (segment (start 138.243 114.3) (end 152.4 114.3) (width 0.2) (layer "B.Cu") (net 4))
 (segment (start 143.892 83.1721) (end 153.288 83.1721) (width 0.2) (layer "B.Cu") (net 4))
 (segment (start 136.793 112.85) (end 138.243 114.3) (width 0.2) (layer "B.Cu") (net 4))
 (segment (start 142.66 81.94) (end 143.892 83.1721) (width 0.2) (layer "B.Cu") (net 4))
 (segment (start 153.288 83.1721) (end 154.52 81.94) (width 0.2) (layer "B.Cu") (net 4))
 (segment (start 136.793 112.85) (end 136.793 114.3) (width 0.2) (layer "B.Cu") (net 4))
 (segment (start 136.793 114.3) (end 136.793 112.85) (width 0.2) (layer "B.Cu") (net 4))
 (segment (start 152.4 114.3) (end 154.94 116.84) (width 0.2) (layer "B.Cu") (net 4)))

